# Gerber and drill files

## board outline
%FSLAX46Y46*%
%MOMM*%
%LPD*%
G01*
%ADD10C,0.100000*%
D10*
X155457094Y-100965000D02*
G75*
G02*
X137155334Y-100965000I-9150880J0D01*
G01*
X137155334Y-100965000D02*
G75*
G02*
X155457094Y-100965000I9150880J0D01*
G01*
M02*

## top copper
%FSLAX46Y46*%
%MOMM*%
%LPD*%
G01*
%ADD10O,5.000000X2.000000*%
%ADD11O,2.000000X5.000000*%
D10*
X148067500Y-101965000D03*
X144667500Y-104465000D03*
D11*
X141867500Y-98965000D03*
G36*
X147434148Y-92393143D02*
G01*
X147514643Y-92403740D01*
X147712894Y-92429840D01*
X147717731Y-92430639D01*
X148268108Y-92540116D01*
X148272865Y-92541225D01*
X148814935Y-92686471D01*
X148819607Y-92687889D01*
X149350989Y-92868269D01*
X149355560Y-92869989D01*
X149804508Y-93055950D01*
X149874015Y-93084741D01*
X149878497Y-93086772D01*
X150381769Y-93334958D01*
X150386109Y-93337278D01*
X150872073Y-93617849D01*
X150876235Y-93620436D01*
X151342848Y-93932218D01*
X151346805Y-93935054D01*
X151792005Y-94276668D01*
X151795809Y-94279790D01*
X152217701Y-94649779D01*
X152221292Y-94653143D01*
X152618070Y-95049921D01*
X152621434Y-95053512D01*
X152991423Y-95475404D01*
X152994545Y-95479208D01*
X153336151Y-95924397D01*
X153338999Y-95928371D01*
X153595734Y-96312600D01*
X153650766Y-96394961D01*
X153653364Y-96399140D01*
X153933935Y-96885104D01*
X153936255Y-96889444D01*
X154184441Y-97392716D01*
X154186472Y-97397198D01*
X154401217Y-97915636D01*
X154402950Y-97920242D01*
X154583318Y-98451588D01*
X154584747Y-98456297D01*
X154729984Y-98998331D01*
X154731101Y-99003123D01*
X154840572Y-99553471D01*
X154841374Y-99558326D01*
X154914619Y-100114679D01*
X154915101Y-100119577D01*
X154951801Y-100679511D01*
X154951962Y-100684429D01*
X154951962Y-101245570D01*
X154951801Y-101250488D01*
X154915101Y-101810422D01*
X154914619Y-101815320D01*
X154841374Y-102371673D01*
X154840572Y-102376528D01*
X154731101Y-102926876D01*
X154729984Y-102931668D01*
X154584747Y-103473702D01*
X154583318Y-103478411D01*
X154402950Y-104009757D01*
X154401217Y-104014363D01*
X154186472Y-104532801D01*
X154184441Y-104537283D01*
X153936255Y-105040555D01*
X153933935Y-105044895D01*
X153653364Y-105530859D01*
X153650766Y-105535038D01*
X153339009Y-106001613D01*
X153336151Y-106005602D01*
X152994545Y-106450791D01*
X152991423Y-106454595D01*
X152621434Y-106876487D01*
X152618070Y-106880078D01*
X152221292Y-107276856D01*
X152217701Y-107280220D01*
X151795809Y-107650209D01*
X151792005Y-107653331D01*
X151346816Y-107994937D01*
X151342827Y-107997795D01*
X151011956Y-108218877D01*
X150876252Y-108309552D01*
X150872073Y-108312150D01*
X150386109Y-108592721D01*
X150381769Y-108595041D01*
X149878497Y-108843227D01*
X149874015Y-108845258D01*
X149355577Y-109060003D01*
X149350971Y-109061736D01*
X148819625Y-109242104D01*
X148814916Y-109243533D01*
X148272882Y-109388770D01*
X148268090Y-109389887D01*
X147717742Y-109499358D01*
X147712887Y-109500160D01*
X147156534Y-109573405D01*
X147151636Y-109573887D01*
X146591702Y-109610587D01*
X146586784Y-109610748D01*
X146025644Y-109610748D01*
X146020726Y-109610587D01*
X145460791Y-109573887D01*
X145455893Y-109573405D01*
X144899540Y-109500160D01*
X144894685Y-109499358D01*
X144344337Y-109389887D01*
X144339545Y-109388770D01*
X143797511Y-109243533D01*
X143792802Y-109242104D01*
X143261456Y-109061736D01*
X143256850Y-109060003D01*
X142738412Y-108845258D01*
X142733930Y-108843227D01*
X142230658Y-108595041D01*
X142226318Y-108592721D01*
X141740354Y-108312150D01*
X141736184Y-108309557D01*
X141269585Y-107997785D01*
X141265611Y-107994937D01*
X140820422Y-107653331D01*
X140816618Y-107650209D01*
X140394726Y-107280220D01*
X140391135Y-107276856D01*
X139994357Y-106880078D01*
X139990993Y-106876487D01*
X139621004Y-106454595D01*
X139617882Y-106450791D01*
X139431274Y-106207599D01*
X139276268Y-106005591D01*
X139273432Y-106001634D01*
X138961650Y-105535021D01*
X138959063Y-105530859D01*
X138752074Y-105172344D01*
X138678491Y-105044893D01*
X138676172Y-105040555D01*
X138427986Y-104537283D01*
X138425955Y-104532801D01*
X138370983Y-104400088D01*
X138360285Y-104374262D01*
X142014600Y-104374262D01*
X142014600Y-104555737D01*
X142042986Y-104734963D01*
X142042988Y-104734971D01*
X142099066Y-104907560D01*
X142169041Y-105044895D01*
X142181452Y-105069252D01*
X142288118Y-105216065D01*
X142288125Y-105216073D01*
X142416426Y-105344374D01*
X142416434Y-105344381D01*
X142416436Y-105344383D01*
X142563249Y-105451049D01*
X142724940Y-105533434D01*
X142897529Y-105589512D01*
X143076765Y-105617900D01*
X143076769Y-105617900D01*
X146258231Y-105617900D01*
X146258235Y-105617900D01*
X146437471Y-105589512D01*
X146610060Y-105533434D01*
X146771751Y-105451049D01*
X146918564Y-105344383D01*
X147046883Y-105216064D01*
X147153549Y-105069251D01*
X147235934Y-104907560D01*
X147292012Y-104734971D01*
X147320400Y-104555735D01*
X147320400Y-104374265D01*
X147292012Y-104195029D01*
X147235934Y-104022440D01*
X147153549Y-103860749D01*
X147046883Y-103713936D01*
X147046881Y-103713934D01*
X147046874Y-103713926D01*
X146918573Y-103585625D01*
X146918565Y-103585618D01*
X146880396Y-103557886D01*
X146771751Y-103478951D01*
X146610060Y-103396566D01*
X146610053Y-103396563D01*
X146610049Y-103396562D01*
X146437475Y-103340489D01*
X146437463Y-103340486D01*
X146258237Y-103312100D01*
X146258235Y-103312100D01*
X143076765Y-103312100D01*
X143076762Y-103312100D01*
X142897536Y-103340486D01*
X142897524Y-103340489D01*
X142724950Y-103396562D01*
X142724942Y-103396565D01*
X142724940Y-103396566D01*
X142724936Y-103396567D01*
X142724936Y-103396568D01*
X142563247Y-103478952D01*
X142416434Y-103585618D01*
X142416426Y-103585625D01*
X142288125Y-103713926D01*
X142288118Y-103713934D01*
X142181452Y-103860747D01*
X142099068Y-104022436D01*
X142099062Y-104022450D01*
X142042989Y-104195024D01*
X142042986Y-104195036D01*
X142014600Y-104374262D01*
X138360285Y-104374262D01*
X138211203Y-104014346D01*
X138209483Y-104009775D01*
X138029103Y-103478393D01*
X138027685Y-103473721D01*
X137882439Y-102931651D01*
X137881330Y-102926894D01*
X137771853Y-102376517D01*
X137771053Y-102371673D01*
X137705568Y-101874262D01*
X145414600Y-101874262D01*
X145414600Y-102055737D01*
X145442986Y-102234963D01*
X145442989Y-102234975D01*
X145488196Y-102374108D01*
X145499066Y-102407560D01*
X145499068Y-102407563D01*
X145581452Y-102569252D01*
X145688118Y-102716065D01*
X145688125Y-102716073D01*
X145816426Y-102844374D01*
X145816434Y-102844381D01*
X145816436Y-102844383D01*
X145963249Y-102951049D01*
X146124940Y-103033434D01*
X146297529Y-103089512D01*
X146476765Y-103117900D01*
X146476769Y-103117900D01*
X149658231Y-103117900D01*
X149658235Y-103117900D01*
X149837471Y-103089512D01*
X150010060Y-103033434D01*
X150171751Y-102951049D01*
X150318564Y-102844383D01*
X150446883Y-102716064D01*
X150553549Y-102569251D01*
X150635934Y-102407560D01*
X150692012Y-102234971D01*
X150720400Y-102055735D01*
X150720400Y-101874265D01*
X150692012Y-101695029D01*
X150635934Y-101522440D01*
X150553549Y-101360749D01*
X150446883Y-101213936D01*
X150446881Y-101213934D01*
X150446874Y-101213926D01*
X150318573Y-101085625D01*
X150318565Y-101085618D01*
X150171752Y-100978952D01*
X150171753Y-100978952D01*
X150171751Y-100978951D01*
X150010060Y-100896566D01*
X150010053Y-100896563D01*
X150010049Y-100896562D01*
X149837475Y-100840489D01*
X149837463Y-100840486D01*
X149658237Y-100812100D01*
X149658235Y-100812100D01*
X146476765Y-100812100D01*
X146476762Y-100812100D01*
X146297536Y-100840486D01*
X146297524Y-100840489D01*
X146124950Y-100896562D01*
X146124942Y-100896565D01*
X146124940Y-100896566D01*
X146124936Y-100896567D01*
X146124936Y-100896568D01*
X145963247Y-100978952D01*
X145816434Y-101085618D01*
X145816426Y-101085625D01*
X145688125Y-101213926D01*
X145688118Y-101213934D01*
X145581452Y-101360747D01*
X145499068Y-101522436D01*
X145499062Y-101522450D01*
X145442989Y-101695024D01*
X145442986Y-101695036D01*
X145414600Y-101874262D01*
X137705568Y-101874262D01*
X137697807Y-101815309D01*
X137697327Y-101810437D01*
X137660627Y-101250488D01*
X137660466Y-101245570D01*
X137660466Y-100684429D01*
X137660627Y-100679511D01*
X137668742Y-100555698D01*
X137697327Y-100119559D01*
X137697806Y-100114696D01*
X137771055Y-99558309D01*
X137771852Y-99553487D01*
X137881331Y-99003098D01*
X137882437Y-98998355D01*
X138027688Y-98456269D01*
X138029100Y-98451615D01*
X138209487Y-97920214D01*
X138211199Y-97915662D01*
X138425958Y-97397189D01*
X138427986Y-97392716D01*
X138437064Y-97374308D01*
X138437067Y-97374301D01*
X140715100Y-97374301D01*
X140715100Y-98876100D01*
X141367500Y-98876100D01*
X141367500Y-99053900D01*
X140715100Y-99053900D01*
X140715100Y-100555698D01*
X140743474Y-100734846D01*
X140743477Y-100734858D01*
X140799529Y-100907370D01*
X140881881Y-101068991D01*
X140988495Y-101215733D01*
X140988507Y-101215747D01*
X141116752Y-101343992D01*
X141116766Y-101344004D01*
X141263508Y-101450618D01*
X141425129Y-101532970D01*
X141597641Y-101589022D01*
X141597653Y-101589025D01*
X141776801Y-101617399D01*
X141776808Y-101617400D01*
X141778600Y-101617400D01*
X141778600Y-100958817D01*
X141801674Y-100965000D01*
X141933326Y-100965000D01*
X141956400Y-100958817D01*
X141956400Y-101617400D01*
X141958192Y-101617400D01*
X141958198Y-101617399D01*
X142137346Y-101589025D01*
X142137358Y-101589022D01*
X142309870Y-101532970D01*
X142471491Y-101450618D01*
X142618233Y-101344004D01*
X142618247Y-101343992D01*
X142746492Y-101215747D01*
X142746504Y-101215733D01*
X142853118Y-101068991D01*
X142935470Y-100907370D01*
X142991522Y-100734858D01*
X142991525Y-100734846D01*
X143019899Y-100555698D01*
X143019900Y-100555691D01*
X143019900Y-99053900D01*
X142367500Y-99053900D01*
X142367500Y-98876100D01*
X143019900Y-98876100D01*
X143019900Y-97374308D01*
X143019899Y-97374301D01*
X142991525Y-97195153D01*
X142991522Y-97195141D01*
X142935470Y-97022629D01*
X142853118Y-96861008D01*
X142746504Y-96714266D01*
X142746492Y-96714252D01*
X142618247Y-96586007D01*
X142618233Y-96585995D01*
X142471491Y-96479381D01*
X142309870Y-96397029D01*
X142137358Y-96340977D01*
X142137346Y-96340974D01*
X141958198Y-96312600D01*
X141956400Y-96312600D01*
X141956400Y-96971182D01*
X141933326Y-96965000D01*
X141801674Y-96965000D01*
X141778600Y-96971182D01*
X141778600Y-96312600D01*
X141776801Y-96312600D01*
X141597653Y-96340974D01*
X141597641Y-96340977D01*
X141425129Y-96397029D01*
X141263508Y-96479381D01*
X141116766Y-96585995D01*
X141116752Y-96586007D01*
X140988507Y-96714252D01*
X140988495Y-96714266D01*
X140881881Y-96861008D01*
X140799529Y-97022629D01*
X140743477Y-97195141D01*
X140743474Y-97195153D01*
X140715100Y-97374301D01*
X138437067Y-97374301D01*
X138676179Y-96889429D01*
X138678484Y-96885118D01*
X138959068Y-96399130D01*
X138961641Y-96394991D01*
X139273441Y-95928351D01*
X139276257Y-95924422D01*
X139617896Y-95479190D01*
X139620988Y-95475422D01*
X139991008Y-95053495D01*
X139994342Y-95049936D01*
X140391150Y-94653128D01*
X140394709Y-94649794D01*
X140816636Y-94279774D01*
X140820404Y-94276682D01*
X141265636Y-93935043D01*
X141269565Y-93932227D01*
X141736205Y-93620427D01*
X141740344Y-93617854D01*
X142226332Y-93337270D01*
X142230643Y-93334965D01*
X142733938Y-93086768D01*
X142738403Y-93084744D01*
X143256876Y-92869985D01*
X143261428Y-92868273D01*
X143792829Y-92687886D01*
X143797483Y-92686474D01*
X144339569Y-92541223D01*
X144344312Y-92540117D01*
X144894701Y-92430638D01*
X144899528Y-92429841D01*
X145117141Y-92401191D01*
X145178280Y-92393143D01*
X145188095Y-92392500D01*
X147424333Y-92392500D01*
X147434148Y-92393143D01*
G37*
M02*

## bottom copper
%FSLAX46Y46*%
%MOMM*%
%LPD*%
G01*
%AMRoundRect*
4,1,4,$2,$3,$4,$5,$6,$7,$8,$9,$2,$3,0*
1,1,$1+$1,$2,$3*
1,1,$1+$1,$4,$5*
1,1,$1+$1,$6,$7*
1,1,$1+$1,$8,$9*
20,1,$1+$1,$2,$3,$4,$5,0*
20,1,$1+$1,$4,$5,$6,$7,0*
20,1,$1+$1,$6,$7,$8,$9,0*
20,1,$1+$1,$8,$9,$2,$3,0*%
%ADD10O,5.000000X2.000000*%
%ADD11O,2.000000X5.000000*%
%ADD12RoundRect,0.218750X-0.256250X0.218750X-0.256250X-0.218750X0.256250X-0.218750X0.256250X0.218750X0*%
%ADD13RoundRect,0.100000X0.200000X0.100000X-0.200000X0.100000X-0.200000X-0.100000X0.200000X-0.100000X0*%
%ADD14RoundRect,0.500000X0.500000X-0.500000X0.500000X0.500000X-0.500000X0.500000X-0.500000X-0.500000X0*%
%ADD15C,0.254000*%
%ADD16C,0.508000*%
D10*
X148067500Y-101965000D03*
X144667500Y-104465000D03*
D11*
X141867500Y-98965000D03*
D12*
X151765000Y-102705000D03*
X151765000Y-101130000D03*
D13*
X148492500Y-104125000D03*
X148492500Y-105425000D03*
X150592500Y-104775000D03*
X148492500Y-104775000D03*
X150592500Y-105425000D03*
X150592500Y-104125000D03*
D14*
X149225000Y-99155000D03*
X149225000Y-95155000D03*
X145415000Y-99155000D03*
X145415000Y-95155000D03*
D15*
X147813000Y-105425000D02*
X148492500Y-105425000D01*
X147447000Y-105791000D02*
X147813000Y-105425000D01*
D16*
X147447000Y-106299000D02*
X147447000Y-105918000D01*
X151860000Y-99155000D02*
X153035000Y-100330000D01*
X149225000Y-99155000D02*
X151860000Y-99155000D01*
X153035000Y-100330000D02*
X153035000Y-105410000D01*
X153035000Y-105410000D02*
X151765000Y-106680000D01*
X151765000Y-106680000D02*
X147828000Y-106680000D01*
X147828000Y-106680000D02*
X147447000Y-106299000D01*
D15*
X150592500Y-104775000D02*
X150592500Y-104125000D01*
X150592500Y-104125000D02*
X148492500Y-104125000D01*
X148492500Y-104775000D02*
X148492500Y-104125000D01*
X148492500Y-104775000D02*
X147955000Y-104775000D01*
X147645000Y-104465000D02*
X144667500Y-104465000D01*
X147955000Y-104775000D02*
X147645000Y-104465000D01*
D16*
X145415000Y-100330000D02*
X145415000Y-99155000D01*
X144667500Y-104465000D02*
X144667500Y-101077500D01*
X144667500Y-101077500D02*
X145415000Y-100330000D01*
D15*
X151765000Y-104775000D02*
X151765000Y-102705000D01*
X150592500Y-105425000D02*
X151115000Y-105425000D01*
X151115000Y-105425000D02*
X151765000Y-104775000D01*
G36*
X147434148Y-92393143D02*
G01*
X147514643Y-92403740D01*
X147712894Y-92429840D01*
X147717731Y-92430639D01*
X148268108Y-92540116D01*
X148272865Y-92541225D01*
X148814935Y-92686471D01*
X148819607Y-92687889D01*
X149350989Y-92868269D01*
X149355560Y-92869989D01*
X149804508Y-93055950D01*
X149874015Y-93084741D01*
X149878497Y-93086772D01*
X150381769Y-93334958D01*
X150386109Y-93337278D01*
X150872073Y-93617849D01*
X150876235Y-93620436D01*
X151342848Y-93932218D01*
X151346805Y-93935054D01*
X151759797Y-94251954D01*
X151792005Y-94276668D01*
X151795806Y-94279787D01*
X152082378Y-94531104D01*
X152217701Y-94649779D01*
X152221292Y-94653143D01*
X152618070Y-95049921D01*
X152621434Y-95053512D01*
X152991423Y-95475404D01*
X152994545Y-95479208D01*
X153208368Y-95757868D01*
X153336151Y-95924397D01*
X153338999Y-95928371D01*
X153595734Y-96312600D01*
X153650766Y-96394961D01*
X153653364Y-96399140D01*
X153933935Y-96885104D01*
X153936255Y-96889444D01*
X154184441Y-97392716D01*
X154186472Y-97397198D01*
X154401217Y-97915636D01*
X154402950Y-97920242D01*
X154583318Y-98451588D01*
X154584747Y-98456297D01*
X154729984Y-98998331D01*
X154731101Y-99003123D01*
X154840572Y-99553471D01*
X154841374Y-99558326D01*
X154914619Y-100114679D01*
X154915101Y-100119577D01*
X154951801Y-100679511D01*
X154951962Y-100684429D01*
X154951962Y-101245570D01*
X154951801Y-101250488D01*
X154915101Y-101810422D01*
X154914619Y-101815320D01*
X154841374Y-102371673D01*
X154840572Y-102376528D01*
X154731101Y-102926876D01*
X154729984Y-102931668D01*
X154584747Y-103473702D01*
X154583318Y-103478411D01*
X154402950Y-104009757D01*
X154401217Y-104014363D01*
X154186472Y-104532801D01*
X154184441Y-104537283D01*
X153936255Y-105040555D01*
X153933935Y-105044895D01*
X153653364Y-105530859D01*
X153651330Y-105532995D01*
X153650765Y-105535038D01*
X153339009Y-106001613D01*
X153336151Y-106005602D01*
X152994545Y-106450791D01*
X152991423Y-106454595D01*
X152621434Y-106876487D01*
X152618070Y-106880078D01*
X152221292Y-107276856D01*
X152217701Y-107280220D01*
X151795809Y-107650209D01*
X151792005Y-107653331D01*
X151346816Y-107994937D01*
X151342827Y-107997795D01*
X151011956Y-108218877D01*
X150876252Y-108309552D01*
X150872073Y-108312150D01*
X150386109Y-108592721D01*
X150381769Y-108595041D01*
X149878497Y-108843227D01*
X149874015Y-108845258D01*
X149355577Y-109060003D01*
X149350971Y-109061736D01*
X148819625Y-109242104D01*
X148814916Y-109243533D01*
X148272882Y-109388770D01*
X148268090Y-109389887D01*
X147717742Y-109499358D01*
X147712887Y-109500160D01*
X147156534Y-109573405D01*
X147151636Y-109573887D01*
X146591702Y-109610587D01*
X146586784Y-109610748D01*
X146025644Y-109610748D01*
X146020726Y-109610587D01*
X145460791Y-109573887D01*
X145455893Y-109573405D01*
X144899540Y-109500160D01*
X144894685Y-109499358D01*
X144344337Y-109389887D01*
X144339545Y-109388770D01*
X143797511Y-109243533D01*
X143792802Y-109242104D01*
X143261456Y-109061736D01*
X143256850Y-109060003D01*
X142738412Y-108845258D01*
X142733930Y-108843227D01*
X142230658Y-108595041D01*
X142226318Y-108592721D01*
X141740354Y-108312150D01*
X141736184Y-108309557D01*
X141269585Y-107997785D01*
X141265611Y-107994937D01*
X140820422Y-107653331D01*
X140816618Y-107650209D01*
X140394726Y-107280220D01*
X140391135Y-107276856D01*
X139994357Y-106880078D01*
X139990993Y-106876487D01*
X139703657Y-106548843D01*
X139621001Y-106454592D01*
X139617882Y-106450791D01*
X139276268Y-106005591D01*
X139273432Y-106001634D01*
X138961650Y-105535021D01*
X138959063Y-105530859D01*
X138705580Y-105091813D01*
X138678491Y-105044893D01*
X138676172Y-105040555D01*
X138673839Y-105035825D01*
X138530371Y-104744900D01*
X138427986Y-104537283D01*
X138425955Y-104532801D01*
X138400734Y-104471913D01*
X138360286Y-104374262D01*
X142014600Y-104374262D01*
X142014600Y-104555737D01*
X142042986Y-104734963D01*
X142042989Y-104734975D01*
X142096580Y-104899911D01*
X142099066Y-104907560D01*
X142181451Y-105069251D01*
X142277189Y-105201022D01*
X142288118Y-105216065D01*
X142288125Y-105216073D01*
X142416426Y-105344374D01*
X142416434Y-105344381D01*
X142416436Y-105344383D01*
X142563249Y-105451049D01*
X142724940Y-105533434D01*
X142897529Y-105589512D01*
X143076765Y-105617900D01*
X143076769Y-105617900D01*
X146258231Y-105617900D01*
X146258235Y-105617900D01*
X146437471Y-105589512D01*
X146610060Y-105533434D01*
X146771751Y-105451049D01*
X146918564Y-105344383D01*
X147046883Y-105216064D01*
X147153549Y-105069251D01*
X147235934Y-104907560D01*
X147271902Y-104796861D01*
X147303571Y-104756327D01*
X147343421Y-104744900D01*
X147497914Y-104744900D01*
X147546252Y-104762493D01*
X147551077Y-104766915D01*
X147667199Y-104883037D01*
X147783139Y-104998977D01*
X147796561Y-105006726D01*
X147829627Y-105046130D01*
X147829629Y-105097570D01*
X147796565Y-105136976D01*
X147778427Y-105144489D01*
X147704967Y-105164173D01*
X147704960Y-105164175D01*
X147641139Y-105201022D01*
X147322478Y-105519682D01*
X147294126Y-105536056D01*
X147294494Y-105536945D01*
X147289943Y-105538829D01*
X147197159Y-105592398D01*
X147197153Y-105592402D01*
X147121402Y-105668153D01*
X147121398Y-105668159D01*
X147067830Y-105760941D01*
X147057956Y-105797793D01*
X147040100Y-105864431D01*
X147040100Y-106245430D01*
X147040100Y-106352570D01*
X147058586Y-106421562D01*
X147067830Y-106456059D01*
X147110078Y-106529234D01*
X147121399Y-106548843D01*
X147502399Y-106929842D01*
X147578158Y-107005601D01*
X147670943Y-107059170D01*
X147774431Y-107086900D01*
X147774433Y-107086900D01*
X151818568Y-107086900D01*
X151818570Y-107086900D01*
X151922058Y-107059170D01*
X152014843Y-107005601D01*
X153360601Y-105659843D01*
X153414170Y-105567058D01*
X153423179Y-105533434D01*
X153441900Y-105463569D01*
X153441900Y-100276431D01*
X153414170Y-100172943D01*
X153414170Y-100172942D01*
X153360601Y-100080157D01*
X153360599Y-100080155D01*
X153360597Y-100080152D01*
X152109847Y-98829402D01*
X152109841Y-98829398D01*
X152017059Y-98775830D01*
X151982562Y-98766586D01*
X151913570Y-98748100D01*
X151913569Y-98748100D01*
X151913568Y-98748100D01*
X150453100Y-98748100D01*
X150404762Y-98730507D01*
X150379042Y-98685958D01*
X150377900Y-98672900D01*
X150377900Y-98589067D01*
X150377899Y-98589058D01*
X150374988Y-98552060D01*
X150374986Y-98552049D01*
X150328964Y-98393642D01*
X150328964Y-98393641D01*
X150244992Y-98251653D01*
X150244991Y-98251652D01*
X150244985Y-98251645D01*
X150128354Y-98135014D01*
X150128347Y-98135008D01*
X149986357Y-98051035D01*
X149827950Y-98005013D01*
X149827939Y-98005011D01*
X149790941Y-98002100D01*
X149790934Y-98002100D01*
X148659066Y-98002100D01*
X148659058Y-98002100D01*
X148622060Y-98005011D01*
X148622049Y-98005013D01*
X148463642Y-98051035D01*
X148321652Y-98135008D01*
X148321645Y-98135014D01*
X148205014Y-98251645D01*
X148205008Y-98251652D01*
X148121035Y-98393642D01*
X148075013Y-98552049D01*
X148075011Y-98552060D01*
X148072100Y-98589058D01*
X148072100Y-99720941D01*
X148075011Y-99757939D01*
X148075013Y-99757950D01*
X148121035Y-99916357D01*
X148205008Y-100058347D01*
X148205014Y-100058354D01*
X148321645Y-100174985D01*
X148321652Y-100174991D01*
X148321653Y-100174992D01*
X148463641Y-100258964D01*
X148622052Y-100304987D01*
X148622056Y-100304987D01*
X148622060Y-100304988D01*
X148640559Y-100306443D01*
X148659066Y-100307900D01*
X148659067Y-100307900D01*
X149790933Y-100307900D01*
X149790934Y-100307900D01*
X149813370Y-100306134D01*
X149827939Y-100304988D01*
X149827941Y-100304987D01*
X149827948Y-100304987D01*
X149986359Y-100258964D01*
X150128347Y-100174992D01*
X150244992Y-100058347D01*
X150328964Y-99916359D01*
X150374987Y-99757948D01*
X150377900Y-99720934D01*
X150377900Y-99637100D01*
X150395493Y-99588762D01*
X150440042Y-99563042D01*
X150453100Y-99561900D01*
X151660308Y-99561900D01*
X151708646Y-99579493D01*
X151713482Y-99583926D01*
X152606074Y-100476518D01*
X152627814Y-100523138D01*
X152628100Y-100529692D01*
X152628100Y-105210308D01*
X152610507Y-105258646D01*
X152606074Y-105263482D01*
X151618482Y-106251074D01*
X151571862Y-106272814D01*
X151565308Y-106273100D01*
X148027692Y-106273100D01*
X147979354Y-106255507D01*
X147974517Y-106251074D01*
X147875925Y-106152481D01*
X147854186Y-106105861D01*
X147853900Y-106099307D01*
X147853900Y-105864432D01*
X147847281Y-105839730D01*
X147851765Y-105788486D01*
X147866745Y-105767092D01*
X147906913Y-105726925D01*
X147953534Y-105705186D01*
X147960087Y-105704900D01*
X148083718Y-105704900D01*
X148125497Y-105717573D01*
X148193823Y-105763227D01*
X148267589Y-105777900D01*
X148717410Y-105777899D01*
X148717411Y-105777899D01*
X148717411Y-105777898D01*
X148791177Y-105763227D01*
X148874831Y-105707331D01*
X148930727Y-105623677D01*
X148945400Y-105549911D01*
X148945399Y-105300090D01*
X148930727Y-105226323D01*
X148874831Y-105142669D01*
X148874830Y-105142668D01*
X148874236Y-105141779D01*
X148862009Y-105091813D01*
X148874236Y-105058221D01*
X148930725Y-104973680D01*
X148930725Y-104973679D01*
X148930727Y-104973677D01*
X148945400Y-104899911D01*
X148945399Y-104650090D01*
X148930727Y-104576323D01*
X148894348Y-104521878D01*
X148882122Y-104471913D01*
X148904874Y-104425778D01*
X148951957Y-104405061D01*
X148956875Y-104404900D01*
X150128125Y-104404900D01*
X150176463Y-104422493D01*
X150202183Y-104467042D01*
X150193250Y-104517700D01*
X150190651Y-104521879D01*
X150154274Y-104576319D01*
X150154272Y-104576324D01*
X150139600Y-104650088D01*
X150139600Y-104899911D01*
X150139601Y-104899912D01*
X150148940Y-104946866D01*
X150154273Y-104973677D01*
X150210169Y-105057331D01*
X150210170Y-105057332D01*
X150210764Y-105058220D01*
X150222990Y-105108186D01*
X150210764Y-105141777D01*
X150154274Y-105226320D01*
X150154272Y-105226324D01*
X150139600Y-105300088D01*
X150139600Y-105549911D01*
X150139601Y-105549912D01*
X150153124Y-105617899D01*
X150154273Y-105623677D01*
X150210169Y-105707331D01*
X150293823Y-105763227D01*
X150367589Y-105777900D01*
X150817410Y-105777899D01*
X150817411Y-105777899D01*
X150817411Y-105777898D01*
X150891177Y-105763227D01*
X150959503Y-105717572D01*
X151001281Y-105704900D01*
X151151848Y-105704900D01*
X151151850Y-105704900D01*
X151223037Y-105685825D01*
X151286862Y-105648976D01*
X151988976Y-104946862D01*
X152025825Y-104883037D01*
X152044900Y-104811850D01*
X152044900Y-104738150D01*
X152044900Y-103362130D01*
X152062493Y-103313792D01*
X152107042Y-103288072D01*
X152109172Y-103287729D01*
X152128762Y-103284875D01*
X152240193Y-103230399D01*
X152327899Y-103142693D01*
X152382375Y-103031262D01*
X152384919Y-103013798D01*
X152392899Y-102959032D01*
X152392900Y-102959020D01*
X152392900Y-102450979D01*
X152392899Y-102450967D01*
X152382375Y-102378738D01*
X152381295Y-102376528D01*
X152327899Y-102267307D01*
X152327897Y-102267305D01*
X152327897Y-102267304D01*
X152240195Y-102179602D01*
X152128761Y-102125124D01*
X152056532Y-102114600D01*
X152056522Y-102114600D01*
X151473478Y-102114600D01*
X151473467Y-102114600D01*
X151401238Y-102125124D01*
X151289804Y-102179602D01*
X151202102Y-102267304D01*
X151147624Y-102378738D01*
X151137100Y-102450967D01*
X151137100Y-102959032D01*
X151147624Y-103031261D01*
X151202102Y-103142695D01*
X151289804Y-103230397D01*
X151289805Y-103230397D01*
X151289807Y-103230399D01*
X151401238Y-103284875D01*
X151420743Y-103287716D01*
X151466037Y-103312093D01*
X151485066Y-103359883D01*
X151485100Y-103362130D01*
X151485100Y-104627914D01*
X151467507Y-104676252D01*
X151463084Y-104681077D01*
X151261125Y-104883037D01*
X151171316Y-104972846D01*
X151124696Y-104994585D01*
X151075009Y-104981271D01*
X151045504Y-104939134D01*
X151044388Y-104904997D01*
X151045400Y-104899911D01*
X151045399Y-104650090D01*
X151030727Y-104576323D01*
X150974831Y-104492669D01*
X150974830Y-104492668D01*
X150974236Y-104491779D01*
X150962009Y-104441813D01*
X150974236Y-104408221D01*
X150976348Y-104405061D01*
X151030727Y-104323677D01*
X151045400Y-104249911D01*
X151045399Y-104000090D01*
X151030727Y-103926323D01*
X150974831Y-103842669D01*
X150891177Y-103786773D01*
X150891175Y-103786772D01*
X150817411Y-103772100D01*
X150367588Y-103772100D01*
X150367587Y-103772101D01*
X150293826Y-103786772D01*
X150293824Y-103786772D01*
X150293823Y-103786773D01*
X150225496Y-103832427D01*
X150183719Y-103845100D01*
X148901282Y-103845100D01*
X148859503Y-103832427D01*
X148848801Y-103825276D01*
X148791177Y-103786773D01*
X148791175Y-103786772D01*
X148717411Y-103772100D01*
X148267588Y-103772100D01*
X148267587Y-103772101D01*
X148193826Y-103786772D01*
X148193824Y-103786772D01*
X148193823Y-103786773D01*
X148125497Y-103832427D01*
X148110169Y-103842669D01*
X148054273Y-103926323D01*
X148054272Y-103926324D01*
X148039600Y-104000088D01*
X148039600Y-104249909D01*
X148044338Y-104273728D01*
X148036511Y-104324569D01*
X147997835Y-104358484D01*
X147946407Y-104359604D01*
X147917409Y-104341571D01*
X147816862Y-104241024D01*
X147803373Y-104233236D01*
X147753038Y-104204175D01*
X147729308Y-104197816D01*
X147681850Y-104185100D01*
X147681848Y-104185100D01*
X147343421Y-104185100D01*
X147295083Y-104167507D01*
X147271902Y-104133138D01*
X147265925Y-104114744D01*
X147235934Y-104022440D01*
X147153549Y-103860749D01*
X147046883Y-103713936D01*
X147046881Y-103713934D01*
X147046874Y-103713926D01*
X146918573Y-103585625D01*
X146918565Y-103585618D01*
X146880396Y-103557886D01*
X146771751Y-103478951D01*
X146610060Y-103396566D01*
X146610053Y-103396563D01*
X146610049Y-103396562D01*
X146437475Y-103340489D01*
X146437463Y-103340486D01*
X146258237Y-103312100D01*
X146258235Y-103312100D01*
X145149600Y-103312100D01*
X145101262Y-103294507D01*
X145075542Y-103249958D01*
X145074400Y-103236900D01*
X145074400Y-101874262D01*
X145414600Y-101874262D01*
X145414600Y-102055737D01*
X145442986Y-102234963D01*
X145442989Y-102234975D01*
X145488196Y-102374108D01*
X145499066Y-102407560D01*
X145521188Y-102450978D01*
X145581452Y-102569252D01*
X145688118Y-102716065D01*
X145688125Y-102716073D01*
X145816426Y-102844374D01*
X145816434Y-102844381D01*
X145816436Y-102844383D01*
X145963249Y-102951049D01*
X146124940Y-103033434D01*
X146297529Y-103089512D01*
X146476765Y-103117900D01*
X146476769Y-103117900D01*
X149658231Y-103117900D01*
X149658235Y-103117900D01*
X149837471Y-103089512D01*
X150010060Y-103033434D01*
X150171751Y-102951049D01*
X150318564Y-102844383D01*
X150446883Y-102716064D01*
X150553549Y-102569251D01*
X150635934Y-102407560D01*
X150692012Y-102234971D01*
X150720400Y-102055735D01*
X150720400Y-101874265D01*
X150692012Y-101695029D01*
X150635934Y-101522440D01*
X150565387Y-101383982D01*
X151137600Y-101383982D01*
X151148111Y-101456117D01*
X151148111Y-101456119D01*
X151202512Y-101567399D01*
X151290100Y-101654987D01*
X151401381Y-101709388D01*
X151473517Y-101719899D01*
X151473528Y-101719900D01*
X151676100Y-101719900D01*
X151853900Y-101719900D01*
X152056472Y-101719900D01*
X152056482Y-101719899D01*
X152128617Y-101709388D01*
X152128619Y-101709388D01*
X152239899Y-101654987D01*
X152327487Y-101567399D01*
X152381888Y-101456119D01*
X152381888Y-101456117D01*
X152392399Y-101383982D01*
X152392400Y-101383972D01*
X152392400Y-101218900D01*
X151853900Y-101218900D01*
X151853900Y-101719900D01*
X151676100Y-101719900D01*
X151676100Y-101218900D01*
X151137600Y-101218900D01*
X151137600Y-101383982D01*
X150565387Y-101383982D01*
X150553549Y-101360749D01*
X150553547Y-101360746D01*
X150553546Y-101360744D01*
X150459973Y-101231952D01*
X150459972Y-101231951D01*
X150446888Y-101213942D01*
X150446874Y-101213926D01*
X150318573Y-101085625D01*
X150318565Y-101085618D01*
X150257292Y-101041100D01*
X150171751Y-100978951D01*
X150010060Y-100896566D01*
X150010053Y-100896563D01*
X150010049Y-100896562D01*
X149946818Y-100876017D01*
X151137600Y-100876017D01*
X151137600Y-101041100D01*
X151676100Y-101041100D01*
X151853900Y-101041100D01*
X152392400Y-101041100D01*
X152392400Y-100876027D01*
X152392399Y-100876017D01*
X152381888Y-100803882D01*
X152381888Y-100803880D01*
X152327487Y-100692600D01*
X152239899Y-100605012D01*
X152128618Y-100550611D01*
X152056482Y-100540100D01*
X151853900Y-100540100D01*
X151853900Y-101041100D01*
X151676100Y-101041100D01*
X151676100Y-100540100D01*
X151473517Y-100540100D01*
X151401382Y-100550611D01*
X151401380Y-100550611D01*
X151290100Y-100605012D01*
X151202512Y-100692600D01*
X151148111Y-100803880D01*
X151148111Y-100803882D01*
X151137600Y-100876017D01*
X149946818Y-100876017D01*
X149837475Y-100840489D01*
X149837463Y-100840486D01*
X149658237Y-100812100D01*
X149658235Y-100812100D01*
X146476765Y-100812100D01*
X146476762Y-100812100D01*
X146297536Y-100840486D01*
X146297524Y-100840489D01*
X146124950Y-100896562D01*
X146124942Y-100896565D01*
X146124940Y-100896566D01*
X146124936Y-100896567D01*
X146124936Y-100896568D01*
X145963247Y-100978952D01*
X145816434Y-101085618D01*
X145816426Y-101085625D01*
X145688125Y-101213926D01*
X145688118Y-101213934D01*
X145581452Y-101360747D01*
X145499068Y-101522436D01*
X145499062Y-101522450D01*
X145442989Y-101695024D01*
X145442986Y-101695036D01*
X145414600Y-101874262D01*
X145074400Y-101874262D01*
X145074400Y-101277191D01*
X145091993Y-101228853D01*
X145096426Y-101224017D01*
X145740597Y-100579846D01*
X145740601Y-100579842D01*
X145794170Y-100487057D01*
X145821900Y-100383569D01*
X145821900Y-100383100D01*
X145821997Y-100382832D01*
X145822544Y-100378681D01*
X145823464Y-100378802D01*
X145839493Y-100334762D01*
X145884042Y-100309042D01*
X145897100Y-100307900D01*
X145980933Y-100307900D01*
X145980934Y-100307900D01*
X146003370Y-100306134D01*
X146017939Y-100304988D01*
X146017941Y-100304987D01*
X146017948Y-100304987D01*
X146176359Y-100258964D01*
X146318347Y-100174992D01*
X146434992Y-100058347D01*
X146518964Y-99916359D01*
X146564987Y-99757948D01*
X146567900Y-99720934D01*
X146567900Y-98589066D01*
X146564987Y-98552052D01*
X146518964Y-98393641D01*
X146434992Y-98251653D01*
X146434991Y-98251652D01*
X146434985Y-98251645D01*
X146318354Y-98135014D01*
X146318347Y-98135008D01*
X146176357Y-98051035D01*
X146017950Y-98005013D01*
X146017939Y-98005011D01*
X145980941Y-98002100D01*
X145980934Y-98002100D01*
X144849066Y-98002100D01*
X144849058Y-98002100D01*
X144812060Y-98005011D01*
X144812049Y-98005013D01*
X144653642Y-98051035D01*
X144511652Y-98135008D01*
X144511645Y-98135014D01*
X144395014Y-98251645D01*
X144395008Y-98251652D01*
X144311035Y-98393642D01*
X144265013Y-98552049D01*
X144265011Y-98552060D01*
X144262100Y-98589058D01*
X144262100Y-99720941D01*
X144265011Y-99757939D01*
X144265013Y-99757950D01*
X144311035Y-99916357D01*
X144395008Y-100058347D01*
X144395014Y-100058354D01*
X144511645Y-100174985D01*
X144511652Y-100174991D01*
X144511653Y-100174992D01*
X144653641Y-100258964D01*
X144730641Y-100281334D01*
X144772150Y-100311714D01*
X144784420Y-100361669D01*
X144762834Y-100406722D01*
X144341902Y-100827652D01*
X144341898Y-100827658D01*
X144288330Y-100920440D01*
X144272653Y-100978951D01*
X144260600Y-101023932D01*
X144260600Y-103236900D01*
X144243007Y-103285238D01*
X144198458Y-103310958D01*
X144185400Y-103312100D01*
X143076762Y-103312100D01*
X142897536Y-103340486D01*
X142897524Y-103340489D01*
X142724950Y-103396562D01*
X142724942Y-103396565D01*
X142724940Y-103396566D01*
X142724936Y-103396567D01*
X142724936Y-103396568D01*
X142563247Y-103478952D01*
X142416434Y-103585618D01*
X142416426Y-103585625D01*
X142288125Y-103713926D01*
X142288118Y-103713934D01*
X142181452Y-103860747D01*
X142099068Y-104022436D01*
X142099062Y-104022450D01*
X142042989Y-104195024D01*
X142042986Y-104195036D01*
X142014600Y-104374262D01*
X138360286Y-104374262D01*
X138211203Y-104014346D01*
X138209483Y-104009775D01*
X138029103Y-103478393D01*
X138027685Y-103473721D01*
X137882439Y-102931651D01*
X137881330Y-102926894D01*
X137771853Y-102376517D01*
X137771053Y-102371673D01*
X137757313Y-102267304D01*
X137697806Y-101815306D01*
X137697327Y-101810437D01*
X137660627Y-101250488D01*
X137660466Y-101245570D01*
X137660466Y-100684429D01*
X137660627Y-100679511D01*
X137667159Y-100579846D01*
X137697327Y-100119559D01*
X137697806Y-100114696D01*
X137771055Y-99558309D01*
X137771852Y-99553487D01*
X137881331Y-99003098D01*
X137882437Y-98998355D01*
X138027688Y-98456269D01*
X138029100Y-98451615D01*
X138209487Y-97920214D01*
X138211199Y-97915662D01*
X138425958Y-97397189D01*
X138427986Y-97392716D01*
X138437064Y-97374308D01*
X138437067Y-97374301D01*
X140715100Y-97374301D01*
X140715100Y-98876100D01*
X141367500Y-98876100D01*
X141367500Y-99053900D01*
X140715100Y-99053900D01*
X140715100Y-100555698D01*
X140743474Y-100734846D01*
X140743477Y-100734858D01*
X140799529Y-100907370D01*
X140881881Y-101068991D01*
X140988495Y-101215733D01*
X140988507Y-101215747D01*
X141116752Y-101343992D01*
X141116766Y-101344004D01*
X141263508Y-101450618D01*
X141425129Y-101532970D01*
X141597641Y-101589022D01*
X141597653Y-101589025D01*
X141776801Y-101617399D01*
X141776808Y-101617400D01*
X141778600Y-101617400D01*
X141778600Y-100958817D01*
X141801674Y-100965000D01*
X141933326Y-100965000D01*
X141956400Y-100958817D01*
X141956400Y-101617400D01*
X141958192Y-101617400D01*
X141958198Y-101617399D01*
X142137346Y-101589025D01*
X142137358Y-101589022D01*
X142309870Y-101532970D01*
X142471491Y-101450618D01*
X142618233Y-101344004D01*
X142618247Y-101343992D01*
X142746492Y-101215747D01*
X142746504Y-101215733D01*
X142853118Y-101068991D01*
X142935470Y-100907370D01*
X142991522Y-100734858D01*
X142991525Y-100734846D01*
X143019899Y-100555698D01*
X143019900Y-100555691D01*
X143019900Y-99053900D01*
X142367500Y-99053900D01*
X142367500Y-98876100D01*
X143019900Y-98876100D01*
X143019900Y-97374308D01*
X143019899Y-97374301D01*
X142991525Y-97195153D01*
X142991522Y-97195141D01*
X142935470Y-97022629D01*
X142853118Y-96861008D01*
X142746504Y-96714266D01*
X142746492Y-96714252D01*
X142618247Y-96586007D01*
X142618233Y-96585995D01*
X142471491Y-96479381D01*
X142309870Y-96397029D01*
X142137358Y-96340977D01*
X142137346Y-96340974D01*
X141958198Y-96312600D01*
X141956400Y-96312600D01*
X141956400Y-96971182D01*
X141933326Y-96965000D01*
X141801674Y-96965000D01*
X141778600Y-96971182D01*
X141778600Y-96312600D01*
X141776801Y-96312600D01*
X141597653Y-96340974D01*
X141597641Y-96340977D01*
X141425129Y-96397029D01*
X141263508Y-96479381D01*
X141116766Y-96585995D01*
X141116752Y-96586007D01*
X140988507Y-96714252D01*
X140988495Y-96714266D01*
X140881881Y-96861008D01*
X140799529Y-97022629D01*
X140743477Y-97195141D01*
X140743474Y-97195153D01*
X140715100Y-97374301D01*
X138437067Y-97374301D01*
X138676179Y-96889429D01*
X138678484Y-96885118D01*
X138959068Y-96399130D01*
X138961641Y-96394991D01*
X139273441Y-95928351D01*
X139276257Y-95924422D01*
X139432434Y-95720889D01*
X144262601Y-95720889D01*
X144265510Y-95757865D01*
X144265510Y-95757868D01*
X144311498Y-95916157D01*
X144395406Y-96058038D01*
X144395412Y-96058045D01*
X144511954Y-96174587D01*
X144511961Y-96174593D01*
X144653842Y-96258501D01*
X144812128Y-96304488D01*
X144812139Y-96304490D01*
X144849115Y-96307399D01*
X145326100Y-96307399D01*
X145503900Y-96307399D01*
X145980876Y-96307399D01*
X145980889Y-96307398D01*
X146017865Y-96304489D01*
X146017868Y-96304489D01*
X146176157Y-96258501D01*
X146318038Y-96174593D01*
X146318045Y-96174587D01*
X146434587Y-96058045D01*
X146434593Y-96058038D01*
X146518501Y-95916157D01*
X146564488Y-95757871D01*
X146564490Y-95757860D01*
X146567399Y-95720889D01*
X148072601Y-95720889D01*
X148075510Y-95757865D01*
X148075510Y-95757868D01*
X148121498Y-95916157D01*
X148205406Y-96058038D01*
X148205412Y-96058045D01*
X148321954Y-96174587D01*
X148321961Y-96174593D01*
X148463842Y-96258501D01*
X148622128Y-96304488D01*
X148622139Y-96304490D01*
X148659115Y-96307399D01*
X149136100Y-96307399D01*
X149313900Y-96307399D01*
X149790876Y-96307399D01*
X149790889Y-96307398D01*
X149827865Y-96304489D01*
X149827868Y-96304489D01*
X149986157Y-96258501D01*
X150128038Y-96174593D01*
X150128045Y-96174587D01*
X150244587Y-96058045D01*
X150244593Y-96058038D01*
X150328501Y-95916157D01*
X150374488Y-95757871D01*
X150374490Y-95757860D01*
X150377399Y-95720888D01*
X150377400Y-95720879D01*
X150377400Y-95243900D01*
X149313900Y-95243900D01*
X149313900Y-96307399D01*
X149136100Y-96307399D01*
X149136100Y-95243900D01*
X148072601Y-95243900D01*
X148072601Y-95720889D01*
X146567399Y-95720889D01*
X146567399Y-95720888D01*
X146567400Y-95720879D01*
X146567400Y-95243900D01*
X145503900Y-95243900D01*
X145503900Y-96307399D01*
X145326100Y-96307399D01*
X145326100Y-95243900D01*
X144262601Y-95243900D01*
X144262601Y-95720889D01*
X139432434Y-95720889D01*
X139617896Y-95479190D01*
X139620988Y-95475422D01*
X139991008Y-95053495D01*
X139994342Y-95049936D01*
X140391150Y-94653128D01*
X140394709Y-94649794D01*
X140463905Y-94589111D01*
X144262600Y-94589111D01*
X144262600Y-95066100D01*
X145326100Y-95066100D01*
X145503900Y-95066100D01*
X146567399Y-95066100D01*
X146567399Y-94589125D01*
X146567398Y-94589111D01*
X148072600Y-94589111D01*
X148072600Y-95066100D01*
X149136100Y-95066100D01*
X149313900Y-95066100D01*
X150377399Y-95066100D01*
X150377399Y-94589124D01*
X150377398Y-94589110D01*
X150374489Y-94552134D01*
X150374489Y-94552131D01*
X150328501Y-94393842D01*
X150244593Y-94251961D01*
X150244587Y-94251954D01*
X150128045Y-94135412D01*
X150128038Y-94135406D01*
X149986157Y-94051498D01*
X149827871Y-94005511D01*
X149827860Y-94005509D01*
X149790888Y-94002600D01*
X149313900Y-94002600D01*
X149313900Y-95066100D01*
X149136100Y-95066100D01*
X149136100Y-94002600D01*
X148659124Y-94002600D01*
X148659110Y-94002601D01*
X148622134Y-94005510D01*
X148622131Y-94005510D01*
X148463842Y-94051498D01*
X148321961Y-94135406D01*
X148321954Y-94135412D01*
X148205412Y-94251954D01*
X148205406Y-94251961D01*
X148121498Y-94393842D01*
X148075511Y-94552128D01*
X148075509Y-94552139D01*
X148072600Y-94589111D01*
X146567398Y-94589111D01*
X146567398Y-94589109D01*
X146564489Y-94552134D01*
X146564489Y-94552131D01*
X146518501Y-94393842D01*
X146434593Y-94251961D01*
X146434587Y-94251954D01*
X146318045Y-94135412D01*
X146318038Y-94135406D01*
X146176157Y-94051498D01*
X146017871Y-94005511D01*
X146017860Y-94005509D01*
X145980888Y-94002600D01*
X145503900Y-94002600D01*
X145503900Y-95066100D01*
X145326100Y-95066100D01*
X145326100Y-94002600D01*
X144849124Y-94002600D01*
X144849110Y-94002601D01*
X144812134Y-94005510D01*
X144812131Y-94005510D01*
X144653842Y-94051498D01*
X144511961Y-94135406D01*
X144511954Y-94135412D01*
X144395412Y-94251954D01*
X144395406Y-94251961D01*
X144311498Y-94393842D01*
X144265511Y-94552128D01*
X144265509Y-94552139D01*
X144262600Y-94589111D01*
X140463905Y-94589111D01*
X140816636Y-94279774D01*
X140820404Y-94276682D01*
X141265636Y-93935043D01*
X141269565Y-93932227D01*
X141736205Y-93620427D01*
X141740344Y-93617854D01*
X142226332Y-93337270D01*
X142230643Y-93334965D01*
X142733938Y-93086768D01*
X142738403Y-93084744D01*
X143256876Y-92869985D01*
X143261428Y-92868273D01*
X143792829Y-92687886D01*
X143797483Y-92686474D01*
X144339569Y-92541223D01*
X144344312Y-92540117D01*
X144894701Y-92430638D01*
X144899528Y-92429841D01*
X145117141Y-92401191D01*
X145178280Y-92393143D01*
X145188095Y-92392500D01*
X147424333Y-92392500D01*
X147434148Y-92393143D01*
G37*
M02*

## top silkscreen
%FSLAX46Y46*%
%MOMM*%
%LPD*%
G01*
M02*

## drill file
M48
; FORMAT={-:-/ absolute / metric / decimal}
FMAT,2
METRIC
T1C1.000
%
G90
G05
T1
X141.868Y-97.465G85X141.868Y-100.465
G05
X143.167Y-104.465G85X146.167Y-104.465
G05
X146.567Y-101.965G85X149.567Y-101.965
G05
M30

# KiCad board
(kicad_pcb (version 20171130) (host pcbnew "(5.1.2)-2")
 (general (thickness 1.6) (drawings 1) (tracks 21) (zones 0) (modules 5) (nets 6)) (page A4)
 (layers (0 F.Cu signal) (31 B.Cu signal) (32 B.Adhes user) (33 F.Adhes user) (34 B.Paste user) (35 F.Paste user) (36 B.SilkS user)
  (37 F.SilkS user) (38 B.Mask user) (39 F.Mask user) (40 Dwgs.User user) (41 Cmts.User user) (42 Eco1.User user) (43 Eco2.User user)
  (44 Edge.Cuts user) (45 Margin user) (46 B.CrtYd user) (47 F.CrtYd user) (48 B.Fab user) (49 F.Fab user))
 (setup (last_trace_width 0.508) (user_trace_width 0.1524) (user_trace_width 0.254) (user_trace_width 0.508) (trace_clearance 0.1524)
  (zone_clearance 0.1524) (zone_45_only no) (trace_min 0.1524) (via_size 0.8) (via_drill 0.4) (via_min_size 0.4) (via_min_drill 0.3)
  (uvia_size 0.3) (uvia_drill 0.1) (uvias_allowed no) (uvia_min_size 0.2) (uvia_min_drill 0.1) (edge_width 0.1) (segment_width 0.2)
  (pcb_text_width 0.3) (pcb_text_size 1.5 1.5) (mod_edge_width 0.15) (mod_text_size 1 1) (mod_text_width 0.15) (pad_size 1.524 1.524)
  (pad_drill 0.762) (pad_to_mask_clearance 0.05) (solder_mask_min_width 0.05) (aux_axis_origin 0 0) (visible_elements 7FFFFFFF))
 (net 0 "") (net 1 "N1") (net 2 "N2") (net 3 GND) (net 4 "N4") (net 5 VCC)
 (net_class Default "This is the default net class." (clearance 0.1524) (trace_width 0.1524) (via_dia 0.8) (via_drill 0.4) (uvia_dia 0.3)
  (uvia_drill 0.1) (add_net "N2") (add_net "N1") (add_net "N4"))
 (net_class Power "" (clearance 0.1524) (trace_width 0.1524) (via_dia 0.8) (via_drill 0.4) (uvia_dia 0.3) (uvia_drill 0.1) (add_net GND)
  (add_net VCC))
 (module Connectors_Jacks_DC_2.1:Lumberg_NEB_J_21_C (layer F.Cu) (at 146.3675 100.965)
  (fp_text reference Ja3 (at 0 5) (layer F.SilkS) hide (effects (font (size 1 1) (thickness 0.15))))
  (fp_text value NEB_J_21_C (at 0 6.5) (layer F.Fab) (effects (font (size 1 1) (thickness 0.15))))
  (pad 3 thru_hole oval (at 1.7 1) (size 5 2) (drill oval 4 1) (layers *.Cu *.Mask) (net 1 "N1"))
  (pad 2 thru_hole oval (at -1.7 3.5) (size 5 2) (drill oval 4 1) (layers *.Cu *.Mask) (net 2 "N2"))
  (pad 1 thru_hole oval (at -4.5 -2) (size 2 5) (drill oval 1 4) (layers *.Cu *.Mask) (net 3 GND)))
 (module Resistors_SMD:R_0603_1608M (layer B.Cu) (at 151.765 101.9175 270)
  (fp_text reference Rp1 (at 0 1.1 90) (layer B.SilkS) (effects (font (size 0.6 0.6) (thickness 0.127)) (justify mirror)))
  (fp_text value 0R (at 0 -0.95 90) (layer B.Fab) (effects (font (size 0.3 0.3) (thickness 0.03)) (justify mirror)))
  (pad 2 smd roundrect (at 0.7875 0 270) (size 0.875 0.95) (layers B.Cu B.Paste B.Mask) (roundrect_rratio 0.25) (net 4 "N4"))
  (pad 1 smd roundrect (at -0.7875 0 270) (size 0.875 0.95) (layers B.Cu B.Paste B.Mask) (roundrect_rratio 0.25) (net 3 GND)))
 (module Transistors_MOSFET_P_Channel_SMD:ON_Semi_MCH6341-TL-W (layer B.Cu) (at 149.5425 104.775 180)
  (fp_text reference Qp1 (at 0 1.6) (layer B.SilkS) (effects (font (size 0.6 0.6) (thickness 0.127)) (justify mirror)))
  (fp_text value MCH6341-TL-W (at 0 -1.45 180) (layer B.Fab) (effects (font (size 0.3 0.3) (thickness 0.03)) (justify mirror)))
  (pad 6 smd roundrect (at 1.05 0.65 180) (size 0.6 0.4) (layers B.Cu B.Paste B.Mask) (roundrect_rratio 0.25) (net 2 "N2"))
  (pad 4 smd roundrect (at 1.05 -0.65 180) (size 0.6 0.4) (layers B.Cu B.Paste B.Mask) (roundrect_rratio 0.25) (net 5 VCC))
  (pad 2 smd roundrect (at -1.05 0 180) (size 0.6 0.4) (layers B.Cu B.Paste B.Mask) (roundrect_rratio 0.25) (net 2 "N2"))
  (pad 5 smd roundrect (at 1.05 0 180) (size 0.6 0.4) (layers B.Cu B.Paste B.Mask) (roundrect_rratio 0.25) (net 2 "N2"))
  (pad 3 smd roundrect (at -1.05 -0.65 180) (size 0.6 0.4) (layers B.Cu B.Paste B.Mask) (roundrect_rratio 0.25) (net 4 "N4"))
  (pad 1 smd roundrect (at -1.05 0.65 180) (size 0.6 0.4) (layers B.Cu B.Paste B.Mask) (roundrect_rratio 0.25) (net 2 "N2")))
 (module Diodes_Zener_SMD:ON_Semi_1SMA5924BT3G (layer B.Cu) (at 149.225 97.155 90)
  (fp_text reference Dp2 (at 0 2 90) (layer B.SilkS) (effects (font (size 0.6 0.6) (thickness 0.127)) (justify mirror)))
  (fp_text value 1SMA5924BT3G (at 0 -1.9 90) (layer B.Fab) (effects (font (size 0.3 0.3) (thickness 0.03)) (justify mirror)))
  (pad 2 smd roundrect (at -2 0 90) (size 2 2) (layers B.Cu B.Paste B.Mask) (roundrect_rratio 0.25) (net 5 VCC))
  (pad 1 smd roundrect (at 2 0 90) (size 2 2) (layers B.Cu B.Paste B.Mask) (roundrect_rratio 0.25) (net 3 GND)))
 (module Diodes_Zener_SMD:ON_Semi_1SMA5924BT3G (layer B.Cu) (at 145.415 97.155 90)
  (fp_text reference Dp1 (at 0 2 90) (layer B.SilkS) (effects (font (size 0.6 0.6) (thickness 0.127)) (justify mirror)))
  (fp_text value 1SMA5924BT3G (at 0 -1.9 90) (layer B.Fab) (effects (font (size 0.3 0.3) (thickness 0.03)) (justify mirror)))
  (pad 2 smd roundrect (at -2 0 90) (size 2 2) (layers B.Cu B.Paste B.Mask) (roundrect_rratio 0.25) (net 2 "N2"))
  (pad 1 smd roundrect (at 2 0 90) (size 2 2) (layers B.Cu B.Paste B.Mask) (roundrect_rratio 0.25) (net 3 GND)))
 (gr_circle (center 146.306214 100.965) (end 154.305 96.52) (layer Edge.Cuts) (width 0.1))
 (segment (start 147.813 105.425) (end 148.4925 105.425) (width 0.254) (layer B.Cu) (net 5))
 (segment (start 147.447 105.791) (end 147.813 105.425) (width 0.254) (layer B.Cu) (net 5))
 (segment (start 147.447 106.299) (end 147.447 105.918) (width 0.508) (layer B.Cu) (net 5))
 (segment (start 151.86 99.155) (end 153.035 100.33) (width 0.508) (layer B.Cu) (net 5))
 (segment (start 149.225 99.155) (end 151.86 99.155) (width 0.508) (layer B.Cu) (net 5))
 (segment (start 153.035 100.33) (end 153.035 105.41) (width 0.508) (layer B.Cu) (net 5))
 (segment (start 153.035 105.41) (end 151.765 106.68) (width 0.508) (layer B.Cu) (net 5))
 (segment (start 151.765 106.68) (end 147.828 106.68) (width 0.508) (layer B.Cu) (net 5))
 (segment (start 147.828 106.68) (end 147.447 106.299) (width 0.508) (layer B.Cu) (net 5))
 (segment (start 150.5925 104.775) (end 150.5925 104.125) (width 0.254) (layer B.Cu) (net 2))
 (segment (start 150.5925 104.125) (end 148.4925 104.125) (width 0.254) (layer B.Cu) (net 2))
 (segment (start 148.4925 104.775) (end 148.4925 104.125) (width 0.254) (layer B.Cu) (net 2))
 (segment (start 148.4925 104.775) (end 147.955 104.775) (width 0.254) (layer B.Cu) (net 2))
 (segment (start 147.645 104.465) (end 144.6675 104.465) (width 0.254) (layer B.Cu) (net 2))
 (segment (start 147.955 104.775) (end 147.645 104.465) (width 0.254) (layer B.Cu) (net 2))
 (segment (start 145.415 100.33) (end 145.415 99.155) (width 0.508) (layer B.Cu) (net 2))
 (segment (start 144.6675 104.465) (end 144.6675 101.0775) (width 0.508) (layer B.Cu) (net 2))
 (segment (start 144.6675 101.0775) (end 145.415 100.33) (width 0.508) (layer B.Cu) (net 2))
 (segment (start 151.765 104.775) (end 151.765 102.705) (width 0.254) (layer B.Cu) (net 4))
 (segment (start 150.5925 105.425) (end 151.115 105.425) (width 0.254) (layer B.Cu) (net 4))
 (segment (start 151.115 105.425) (end 151.765 104.775) (width 0.254) (layer B.Cu) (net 4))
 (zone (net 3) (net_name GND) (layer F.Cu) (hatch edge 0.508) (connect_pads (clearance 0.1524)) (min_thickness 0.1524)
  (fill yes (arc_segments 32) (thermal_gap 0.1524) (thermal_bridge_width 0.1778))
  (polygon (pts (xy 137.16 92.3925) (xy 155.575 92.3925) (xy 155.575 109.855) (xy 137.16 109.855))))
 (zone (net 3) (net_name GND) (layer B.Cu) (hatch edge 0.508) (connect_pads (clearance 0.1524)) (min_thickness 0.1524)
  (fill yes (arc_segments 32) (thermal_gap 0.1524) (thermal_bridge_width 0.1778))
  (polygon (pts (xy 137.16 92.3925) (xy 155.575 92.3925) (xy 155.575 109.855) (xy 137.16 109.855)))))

